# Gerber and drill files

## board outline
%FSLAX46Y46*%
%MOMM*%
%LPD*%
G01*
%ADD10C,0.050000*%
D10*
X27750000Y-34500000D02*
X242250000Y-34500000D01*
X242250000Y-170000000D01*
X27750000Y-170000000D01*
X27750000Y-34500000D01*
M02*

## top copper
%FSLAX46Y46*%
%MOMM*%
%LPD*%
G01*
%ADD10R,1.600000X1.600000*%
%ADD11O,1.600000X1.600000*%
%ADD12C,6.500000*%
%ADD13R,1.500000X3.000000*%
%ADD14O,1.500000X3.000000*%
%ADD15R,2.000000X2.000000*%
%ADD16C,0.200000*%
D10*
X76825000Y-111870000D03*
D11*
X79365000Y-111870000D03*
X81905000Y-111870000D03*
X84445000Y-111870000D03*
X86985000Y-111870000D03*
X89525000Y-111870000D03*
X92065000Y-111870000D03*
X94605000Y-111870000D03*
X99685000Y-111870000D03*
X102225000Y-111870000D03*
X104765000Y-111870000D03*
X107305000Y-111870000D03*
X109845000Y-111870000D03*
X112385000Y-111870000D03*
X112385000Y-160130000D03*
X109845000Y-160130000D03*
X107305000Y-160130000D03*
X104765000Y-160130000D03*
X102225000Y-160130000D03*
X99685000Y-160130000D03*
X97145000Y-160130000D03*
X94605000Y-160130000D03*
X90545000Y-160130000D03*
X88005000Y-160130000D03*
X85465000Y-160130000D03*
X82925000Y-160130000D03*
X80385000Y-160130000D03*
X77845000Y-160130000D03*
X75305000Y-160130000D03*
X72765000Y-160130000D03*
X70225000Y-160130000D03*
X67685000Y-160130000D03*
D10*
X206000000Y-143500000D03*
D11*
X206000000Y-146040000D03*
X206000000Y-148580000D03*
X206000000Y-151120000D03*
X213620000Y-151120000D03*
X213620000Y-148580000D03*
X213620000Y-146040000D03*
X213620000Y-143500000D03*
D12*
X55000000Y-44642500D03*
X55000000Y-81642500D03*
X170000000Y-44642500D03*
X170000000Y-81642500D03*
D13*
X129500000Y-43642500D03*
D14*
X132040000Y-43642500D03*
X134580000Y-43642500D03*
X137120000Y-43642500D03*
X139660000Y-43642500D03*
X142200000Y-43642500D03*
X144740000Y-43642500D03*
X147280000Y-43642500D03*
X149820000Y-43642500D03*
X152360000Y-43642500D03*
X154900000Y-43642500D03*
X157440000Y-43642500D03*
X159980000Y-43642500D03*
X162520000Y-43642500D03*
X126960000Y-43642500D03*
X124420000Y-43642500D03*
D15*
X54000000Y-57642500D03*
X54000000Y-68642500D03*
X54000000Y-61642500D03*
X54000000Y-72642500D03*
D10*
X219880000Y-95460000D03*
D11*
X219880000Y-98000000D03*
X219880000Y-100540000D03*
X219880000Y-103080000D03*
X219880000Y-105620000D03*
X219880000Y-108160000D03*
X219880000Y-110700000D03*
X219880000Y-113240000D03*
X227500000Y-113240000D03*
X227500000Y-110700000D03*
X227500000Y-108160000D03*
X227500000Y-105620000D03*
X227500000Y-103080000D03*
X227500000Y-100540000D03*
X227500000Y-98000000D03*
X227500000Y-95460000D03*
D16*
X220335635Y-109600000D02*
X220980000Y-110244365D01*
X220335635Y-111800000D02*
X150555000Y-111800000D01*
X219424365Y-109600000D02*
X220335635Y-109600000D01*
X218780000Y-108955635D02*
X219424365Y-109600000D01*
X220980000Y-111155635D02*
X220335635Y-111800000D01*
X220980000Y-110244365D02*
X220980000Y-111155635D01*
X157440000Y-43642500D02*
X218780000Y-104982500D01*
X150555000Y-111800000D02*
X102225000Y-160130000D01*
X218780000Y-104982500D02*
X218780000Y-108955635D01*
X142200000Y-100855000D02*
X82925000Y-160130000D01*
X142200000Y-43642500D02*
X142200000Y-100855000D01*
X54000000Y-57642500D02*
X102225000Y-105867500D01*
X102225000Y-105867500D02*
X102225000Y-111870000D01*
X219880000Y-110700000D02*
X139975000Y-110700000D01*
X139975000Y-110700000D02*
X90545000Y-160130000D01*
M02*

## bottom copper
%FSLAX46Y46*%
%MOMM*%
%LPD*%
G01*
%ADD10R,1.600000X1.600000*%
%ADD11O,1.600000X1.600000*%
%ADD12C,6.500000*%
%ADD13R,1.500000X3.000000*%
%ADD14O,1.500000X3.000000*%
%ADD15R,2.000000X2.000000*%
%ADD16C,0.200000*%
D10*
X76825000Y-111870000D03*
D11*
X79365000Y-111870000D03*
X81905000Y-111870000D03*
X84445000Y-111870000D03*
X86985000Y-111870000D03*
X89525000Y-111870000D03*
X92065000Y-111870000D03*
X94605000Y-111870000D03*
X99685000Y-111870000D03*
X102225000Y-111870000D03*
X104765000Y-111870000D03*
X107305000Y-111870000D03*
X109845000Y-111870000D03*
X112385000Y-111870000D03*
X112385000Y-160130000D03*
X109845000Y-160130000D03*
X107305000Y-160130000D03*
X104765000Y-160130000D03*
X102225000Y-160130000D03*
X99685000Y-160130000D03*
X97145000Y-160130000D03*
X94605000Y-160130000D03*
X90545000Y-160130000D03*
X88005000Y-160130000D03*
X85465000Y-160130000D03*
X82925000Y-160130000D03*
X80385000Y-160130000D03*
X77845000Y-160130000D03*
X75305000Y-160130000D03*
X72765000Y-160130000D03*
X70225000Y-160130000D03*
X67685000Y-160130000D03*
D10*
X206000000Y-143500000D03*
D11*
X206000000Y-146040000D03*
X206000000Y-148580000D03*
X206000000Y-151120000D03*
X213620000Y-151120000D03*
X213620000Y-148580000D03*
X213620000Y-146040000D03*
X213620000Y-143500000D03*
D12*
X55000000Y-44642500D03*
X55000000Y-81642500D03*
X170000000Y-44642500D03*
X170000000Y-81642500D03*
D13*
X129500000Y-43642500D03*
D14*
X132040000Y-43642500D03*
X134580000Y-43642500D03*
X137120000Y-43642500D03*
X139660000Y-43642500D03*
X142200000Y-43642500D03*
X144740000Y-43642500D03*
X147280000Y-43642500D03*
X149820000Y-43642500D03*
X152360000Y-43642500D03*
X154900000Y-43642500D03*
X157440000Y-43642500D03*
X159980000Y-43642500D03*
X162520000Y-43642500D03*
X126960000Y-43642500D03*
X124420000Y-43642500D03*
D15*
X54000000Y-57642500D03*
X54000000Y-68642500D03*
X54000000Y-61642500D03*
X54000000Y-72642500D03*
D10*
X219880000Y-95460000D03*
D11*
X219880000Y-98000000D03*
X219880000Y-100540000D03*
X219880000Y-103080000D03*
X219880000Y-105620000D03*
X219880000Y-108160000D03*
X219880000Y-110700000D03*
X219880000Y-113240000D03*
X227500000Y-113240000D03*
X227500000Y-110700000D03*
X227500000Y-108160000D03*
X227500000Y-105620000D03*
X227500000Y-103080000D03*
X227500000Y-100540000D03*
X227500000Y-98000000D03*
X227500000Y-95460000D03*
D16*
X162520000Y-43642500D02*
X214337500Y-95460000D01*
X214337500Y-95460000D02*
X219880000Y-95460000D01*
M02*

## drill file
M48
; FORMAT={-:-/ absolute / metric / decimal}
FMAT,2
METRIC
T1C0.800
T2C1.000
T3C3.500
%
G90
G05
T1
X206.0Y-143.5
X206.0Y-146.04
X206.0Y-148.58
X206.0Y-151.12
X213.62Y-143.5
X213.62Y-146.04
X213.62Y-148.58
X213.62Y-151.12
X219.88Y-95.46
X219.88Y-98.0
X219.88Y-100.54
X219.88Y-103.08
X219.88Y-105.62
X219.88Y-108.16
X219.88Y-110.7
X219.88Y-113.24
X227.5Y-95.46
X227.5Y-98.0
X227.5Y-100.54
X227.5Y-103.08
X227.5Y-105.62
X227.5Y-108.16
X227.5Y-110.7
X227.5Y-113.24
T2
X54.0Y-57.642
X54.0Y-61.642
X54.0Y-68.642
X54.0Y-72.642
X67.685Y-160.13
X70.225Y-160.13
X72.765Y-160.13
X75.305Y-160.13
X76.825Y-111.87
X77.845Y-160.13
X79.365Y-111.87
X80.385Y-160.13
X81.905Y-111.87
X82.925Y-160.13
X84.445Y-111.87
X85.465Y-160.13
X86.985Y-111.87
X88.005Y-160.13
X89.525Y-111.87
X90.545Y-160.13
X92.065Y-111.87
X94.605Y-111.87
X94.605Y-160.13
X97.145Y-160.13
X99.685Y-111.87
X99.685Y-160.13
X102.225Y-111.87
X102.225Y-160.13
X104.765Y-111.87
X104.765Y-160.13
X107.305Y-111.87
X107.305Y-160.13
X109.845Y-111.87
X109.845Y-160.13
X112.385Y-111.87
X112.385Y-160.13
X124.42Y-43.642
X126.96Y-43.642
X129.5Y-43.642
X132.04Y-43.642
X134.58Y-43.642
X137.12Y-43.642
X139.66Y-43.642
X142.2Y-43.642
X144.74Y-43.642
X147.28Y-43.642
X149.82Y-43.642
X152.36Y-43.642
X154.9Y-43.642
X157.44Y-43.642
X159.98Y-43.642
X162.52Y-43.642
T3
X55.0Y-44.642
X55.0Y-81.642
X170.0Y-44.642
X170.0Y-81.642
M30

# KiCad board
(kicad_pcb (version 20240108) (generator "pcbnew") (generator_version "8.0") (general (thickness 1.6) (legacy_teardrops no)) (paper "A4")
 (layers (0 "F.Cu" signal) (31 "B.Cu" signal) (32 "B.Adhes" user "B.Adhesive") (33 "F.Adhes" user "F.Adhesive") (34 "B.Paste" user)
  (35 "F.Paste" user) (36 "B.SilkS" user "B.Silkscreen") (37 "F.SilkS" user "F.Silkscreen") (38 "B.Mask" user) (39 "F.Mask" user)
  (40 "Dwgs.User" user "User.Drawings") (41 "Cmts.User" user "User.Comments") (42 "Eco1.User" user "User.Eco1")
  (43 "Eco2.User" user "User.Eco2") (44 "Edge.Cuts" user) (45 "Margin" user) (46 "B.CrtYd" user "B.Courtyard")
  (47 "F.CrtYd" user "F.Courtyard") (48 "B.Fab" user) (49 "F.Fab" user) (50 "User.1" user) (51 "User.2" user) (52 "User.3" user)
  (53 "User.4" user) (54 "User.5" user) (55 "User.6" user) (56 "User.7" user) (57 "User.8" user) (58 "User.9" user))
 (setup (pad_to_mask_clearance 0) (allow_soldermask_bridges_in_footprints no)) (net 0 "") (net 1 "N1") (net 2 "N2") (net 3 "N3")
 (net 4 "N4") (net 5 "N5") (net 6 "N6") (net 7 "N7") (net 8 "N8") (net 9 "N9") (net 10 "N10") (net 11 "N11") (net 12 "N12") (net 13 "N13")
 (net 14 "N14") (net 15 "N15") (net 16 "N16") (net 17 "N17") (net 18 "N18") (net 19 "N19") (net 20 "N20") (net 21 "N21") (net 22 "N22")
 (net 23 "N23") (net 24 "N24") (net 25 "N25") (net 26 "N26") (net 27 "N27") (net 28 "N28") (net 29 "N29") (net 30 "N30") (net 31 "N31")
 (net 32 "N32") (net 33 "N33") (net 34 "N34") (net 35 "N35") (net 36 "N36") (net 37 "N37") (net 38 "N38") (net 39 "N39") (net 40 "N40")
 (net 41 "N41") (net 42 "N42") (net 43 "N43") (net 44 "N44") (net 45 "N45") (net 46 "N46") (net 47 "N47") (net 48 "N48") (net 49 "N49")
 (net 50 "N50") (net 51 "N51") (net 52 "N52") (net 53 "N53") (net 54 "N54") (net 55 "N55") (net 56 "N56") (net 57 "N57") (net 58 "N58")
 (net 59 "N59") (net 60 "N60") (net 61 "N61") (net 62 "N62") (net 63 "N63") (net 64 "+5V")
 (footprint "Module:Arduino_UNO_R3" (layer "F.Cu") (at 76.825 111.87)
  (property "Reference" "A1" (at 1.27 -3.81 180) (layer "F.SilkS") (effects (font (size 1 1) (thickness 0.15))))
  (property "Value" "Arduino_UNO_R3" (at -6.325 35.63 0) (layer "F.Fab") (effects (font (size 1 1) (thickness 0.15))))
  (pad "1" thru_hole rect (at 0 0 90) (size 1.6 1.6) (drill 1) (layers "*.Cu" "*.Mask") (remove_unused_layers no) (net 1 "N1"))
  (pad "2" thru_hole oval (at 2.54 0 90) (size 1.6 1.6) (drill 1) (layers "*.Cu" "*.Mask") (remove_unused_layers no) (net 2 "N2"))
  (pad "3" thru_hole oval (at 5.08 0 90) (size 1.6 1.6) (drill 1) (layers "*.Cu" "*.Mask") (remove_unused_layers no) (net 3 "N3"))
  (pad "4" thru_hole oval (at 7.62 0 90) (size 1.6 1.6) (drill 1) (layers "*.Cu" "*.Mask") (remove_unused_layers no) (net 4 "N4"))
  (pad "5" thru_hole oval (at 10.16 0 90) (size 1.6 1.6) (drill 1) (layers "*.Cu" "*.Mask") (remove_unused_layers no) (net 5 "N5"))
  (pad "6" thru_hole oval (at 12.7 0 90) (size 1.6 1.6) (drill 1) (layers "*.Cu" "*.Mask") (remove_unused_layers no) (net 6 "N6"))
  (pad "7" thru_hole oval (at 15.24 0 90) (size 1.6 1.6) (drill 1) (layers "*.Cu" "*.Mask") (remove_unused_layers no) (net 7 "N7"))
  (pad "8" thru_hole oval (at 17.78 0 90) (size 1.6 1.6) (drill 1) (layers "*.Cu" "*.Mask") (remove_unused_layers no) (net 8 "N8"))
  (pad "9" thru_hole oval (at 22.86 0 90) (size 1.6 1.6) (drill 1) (layers "*.Cu" "*.Mask") (remove_unused_layers no) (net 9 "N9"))
  (pad "10" thru_hole oval (at 25.4 0 90) (size 1.6 1.6) (drill 1) (layers "*.Cu" "*.Mask") (remove_unused_layers no) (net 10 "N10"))
  (pad "11" thru_hole oval (at 27.94 0 90) (size 1.6 1.6) (drill 1) (layers "*.Cu" "*.Mask") (remove_unused_layers no) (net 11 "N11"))
  (pad "12" thru_hole oval (at 30.48 0 90) (size 1.6 1.6) (drill 1) (layers "*.Cu" "*.Mask") (remove_unused_layers no) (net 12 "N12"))
  (pad "13" thru_hole oval (at 33.02 0 90) (size 1.6 1.6) (drill 1) (layers "*.Cu" "*.Mask") (remove_unused_layers no) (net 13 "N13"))
  (pad "14" thru_hole oval (at 35.56 0 90) (size 1.6 1.6) (drill 1) (layers "*.Cu" "*.Mask") (remove_unused_layers no) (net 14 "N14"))
  (pad "15" thru_hole oval (at 35.56 48.26 90) (size 1.6 1.6) (drill 1) (layers "*.Cu" "*.Mask") (remove_unused_layers no) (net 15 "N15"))
  (pad "16" thru_hole oval (at 33.02 48.26 90) (size 1.6 1.6) (drill 1) (layers "*.Cu" "*.Mask") (remove_unused_layers no) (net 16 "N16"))
  (pad "17" thru_hole oval (at 30.48 48.26 90) (size 1.6 1.6) (drill 1) (layers "*.Cu" "*.Mask") (remove_unused_layers no) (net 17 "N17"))
  (pad "18" thru_hole oval (at 27.94 48.26 90) (size 1.6 1.6) (drill 1) (layers "*.Cu" "*.Mask") (remove_unused_layers no) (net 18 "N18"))
  (pad "19" thru_hole oval (at 25.4 48.26 90) (size 1.6 1.6) (drill 1) (layers "*.Cu" "*.Mask") (remove_unused_layers no) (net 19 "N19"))
  (pad "20" thru_hole oval (at 22.86 48.26 90) (size 1.6 1.6) (drill 1) (layers "*.Cu" "*.Mask") (remove_unused_layers no) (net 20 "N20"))
  (pad "21" thru_hole oval (at 20.32 48.26 90) (size 1.6 1.6) (drill 1) (layers "*.Cu" "*.Mask") (remove_unused_layers no) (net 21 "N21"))
  (pad "22" thru_hole oval (at 17.78 48.26 90) (size 1.6 1.6) (drill 1) (layers "*.Cu" "*.Mask") (remove_unused_layers no) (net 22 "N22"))
  (pad "23" thru_hole oval (at 13.72 48.26 90) (size 1.6 1.6) (drill 1) (layers "*.Cu" "*.Mask") (remove_unused_layers no) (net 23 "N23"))
  (pad "24" thru_hole oval (at 11.18 48.26 90) (size 1.6 1.6) (drill 1) (layers "*.Cu" "*.Mask") (remove_unused_layers no) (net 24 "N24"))
  (pad "25" thru_hole oval (at 8.64 48.26 90) (size 1.6 1.6) (drill 1) (layers "*.Cu" "*.Mask") (remove_unused_layers no) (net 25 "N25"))
  (pad "26" thru_hole oval (at 6.1 48.26 90) (size 1.6 1.6) (drill 1) (layers "*.Cu" "*.Mask") (remove_unused_layers no) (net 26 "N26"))
  (pad "27" thru_hole oval (at 3.56 48.26 90) (size 1.6 1.6) (drill 1) (layers "*.Cu" "*.Mask") (remove_unused_layers no) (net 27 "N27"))
  (pad "28" thru_hole oval (at 1.02 48.26 90) (size 1.6 1.6) (drill 1) (layers "*.Cu" "*.Mask") (remove_unused_layers no) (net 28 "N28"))
  (pad "29" thru_hole oval (at -1.52 48.26 90) (size 1.6 1.6) (drill 1) (layers "*.Cu" "*.Mask") (remove_unused_layers no) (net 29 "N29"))
  (pad "30" thru_hole oval (at -4.06 48.26 90) (size 1.6 1.6) (drill 1) (layers "*.Cu" "*.Mask") (remove_unused_layers no) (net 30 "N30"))
  (pad "31" thru_hole oval (at -6.6 48.26 90) (size 1.6 1.6) (drill 1) (layers "*.Cu" "*.Mask") (remove_unused_layers no) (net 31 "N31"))
  (pad "32" thru_hole oval (at -9.14 48.26 90) (size 1.6 1.6) (drill 1) (layers "*.Cu" "*.Mask") (remove_unused_layers no) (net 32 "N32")))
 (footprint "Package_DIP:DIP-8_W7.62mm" (layer "F.Cu") (at 206 143.5)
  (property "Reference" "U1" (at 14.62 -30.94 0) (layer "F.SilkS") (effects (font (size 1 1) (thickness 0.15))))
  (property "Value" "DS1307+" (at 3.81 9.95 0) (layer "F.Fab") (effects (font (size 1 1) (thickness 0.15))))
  (pad "1" thru_hole rect (at 0 0) (size 1.6 1.6) (drill 0.8) (layers "*.Cu" "*.Mask") (remove_unused_layers no) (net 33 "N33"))
  (pad "2" thru_hole oval (at 0 2.54) (size 1.6 1.6) (drill 0.8) (layers "*.Cu" "*.Mask") (remove_unused_layers no) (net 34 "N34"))
  (pad "3" thru_hole oval (at 0 5.08) (size 1.6 1.6) (drill 0.8) (layers "*.Cu" "*.Mask") (remove_unused_layers no) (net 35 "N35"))
  (pad "4" thru_hole oval (at 0 7.62) (size 1.6 1.6) (drill 0.8) (layers "*.Cu" "*.Mask") (remove_unused_layers no) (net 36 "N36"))
  (pad "5" thru_hole oval (at 7.62 7.62) (size 1.6 1.6) (drill 0.8) (layers "*.Cu" "*.Mask") (remove_unused_layers no) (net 13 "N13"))
  (pad "6" thru_hole oval (at 7.62 5.08) (size 1.6 1.6) (drill 0.8) (layers "*.Cu" "*.Mask") (remove_unused_layers no) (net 14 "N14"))
  (pad "7" thru_hole oval (at 7.62 2.54) (size 1.6 1.6) (drill 0.8) (layers "*.Cu" "*.Mask") (remove_unused_layers no) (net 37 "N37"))
  (pad "8" thru_hole oval (at 7.62 0) (size 1.6 1.6) (drill 0.8) (layers "*.Cu" "*.Mask") (remove_unused_layers no) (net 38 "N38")))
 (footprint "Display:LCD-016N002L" (layer "F.Cu") (at 129.5 43.6425)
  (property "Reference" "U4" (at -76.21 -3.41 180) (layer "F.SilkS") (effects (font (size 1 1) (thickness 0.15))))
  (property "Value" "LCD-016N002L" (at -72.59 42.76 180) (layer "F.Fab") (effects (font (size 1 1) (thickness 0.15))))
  (pad "" thru_hole circle (at -74.5 1 180) (size 6.5 6.5) (drill 3.5) (layers "*.Cu" "*.Mask") (remove_unused_layers no))
  (pad "" thru_hole circle (at -74.5 38 180) (size 6.5 6.5) (drill 3.5) (layers "*.Cu" "*.Mask") (remove_unused_layers no))
  (pad "" thru_hole circle (at 40.5 1 180) (size 6.5 6.5) (drill 3.5) (layers "*.Cu" "*.Mask") (remove_unused_layers no))
  (pad "" thru_hole circle (at 40.5 38 180) (size 6.5 6.5) (drill 3.5) (layers "*.Cu" "*.Mask") (remove_unused_layers no))
  (pad "1" thru_hole rect (at 0 0 180) (size 1.5 3) (drill 1) (layers "*.Cu" "*.Mask") (remove_unused_layers no) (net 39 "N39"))
  (pad "2" thru_hole oval (at 2.54 0 180) (size 1.5 3) (drill 1) (layers "*.Cu" "*.Mask") (remove_unused_layers no) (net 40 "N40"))
  (pad "3" thru_hole oval (at 5.08 0 180) (size 1.5 3) (drill 1) (layers "*.Cu" "*.Mask") (remove_unused_layers no) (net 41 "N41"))
  (pad "4" thru_hole oval (at 7.62 0 180) (size 1.5 3) (drill 1) (layers "*.Cu" "*.Mask") (remove_unused_layers no) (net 27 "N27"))
  (pad "5" thru_hole oval (at 10.16 0 180) (size 1.5 3) (drill 1) (layers "*.Cu" "*.Mask") (remove_unused_layers no) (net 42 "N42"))
  (pad "6" thru_hole oval (at 12.7 0 180) (size 1.5 3) (drill 1) (layers "*.Cu" "*.Mask") (remove_unused_layers no) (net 26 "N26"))
  (pad "7" thru_hole oval (at 15.24 0 180) (size 1.5 3) (drill 1) (layers "*.Cu" "*.Mask") (remove_unused_layers no) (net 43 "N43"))
  (pad "8" thru_hole oval (at 17.78 0 180) (size 1.5 3) (drill 1) (layers "*.Cu" "*.Mask") (remove_unused_layers no) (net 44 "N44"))
  (pad "9" thru_hole oval (at 20.32 0 180) (size 1.5 3) (drill 1) (layers "*.Cu" "*.Mask") (remove_unused_layers no) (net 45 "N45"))
  (pad "10" thru_hole oval (at 22.86 0 180) (size 1.5 3) (drill 1) (layers "*.Cu" "*.Mask") (remove_unused_layers no) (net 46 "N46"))
  (pad "11" thru_hole oval (at 25.4 0 180) (size 1.5 3) (drill 1) (layers "*.Cu" "*.Mask") (remove_unused_layers no) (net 20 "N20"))
  (pad "12" thru_hole oval (at 27.94 0 180) (size 1.5 3) (drill 1) (layers "*.Cu" "*.Mask") (remove_unused_layers no) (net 19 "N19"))
  (pad "13" thru_hole oval (at 30.48 0 180) (size 1.5 3) (drill 1) (layers "*.Cu" "*.Mask") (remove_unused_layers no) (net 18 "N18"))
  (pad "14" thru_hole oval (at 33.02 0 180) (size 1.5 3) (drill 1) (layers "*.Cu" "*.Mask") (remove_unused_layers no) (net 17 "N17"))
  (pad "15" thru_hole oval (at -2.54 0 180) (size 1.5 3) (drill 1) (layers "*.Cu" "*.Mask") (remove_unused_layers no) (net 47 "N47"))
  (pad "16" thru_hole oval (at -5.08 0 180) (size 1.5 3) (drill 1) (layers "*.Cu" "*.Mask") (remove_unused_layers no) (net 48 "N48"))
  (pad "A1" thru_hole rect (at -75.5 14 180) (size 2 2) (drill 1) (layers "*.Cu" "*.Mask") (remove_unused_layers no) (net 10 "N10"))
  (pad "A2" thru_hole rect (at -75.5 25 180) (size 2 2) (drill 1) (layers "*.Cu" "*.Mask") (remove_unused_layers no) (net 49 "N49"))
  (pad "K1" thru_hole rect (at -75.5 18 180) (size 2 2) (drill 1) (layers "*.Cu" "*.Mask") (remove_unused_layers no) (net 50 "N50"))
  (pad "K2" thru_hole rect (at -75.5 29 180) (size 2 2) (drill 1) (layers "*.Cu" "*.Mask") (remove_unused_layers no) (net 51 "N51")))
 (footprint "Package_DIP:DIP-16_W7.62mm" (layer "F.Cu") (at 219.88 95.46)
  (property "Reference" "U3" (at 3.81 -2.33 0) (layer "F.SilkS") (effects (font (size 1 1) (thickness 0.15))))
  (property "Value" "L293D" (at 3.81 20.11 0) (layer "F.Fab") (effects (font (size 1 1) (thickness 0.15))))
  (pad "1" thru_hole rect (at 0 0) (size 1.6 1.6) (drill 0.8) (layers "*.Cu" "*.Mask") (remove_unused_layers no) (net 17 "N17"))
  (pad "2" thru_hole oval (at 0 2.54) (size 1.6 1.6) (drill 0.8) (layers "*.Cu" "*.Mask") (remove_unused_layers no) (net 24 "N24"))
  (pad "3" thru_hole oval (at 0 5.08) (size 1.6 1.6) (drill 0.8) (layers "*.Cu" "*.Mask") (remove_unused_layers no) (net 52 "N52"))
  (pad "4" thru_hole oval (at 0 7.62) (size 1.6 1.6) (drill 0.8) (layers "*.Cu" "*.Mask") (remove_unused_layers no) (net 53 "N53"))
  (pad "5" thru_hole oval (at 0 10.16) (size 1.6 1.6) (drill 0.8) (layers "*.Cu" "*.Mask") (remove_unused_layers no) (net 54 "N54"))
  (pad "6" thru_hole oval (at 0 12.7) (size 1.6 1.6) (drill 0.8) (layers "*.Cu" "*.Mask") (remove_unused_layers no) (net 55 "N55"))
  (pad "7" thru_hole oval (at 0 15.24) (size 1.6 1.6) (drill 0.8) (layers "*.Cu" "*.Mask") (remove_unused_layers no) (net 23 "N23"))
  (pad "8" thru_hole oval (at 0 17.78) (size 1.6 1.6) (drill 0.8) (layers "*.Cu" "*.Mask") (remove_unused_layers no) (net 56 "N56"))
  (pad "9" thru_hole oval (at 7.62 17.78) (size 1.6 1.6) (drill 0.8) (layers "*.Cu" "*.Mask") (remove_unused_layers no) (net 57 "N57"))
  (pad "10" thru_hole oval (at 7.62 15.24) (size 1.6 1.6) (drill 0.8) (layers "*.Cu" "*.Mask") (remove_unused_layers no) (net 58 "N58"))
  (pad "11" thru_hole oval (at 7.62 12.7) (size 1.6 1.6) (drill 0.8) (layers "*.Cu" "*.Mask") (remove_unused_layers no) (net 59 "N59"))
  (pad "12" thru_hole oval (at 7.62 10.16) (size 1.6 1.6) (drill 0.8) (layers "*.Cu" "*.Mask") (remove_unused_layers no) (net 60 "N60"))
  (pad "13" thru_hole oval (at 7.62 7.62) (size 1.6 1.6) (drill 0.8) (layers "*.Cu" "*.Mask") (remove_unused_layers no) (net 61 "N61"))
  (pad "14" thru_hole oval (at 7.62 5.08) (size 1.6 1.6) (drill 0.8) (layers "*.Cu" "*.Mask") (remove_unused_layers no) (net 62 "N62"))
  (pad "15" thru_hole oval (at 7.62 2.54) (size 1.6 1.6) (drill 0.8) (layers "*.Cu" "*.Mask") (remove_unused_layers no) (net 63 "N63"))
  (pad "16" thru_hole oval (at 7.62 0) (size 1.6 1.6) (drill 0.8) (layers "*.Cu" "*.Mask") (remove_unused_layers no) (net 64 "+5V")))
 (gr_rect (start 27.75 34.5) (end 242.25 170) (stroke (width 0.05) (type default)) (fill none) (layer "Edge.Cuts"))
 (segment (start 220.335635 109.6) (end 220.98 110.244365) (width 0.2) (layer "F.Cu") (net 19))
 (segment (start 220.335635 111.8) (end 150.555 111.8) (width 0.2) (layer "F.Cu") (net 19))
 (segment (start 219.424365 109.6) (end 220.335635 109.6) (width 0.2) (layer "F.Cu") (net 19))
 (segment (start 218.78 108.955635) (end 219.424365 109.6) (width 0.2) (layer "F.Cu") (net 19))
 (segment (start 220.98 111.155635) (end 220.335635 111.8) (width 0.2) (layer "F.Cu") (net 19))
 (segment (start 220.98 110.244365) (end 220.98 111.155635) (width 0.2) (layer "F.Cu") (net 19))
 (segment (start 157.44 43.6425) (end 218.78 104.9825) (width 0.2) (layer "F.Cu") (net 19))
 (segment (start 150.555 111.8) (end 102.225 160.13) (width 0.2) (layer "F.Cu") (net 19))
 (segment (start 218.78 104.9825) (end 218.78 108.955635) (width 0.2) (layer "F.Cu") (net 19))
 (segment (start 162.52 43.6425) (end 214.3375 95.46) (width 0.2) (layer "B.Cu") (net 17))
 (segment (start 214.3375 95.46) (end 219.88 95.46) (width 0.2) (layer "B.Cu") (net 17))
 (segment (start 142.2 100.855) (end 82.925 160.13) (width 0.2) (layer "F.Cu") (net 26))
 (segment (start 142.2 43.6425) (end 142.2 100.855) (width 0.2) (layer "F.Cu") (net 26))
 (segment (start 54 57.6425) (end 102.225 105.8675) (width 0.2) (layer "F.Cu") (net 10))
 (segment (start 102.225 105.8675) (end 102.225 111.87) (width 0.2) (layer "F.Cu") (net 10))
 (segment (start 219.88 110.7) (end 139.975 110.7) (width 0.2) (layer "F.Cu") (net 23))
 (segment (start 139.975 110.7) (end 90.545 160.13) (width 0.2) (layer "F.Cu") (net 23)))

